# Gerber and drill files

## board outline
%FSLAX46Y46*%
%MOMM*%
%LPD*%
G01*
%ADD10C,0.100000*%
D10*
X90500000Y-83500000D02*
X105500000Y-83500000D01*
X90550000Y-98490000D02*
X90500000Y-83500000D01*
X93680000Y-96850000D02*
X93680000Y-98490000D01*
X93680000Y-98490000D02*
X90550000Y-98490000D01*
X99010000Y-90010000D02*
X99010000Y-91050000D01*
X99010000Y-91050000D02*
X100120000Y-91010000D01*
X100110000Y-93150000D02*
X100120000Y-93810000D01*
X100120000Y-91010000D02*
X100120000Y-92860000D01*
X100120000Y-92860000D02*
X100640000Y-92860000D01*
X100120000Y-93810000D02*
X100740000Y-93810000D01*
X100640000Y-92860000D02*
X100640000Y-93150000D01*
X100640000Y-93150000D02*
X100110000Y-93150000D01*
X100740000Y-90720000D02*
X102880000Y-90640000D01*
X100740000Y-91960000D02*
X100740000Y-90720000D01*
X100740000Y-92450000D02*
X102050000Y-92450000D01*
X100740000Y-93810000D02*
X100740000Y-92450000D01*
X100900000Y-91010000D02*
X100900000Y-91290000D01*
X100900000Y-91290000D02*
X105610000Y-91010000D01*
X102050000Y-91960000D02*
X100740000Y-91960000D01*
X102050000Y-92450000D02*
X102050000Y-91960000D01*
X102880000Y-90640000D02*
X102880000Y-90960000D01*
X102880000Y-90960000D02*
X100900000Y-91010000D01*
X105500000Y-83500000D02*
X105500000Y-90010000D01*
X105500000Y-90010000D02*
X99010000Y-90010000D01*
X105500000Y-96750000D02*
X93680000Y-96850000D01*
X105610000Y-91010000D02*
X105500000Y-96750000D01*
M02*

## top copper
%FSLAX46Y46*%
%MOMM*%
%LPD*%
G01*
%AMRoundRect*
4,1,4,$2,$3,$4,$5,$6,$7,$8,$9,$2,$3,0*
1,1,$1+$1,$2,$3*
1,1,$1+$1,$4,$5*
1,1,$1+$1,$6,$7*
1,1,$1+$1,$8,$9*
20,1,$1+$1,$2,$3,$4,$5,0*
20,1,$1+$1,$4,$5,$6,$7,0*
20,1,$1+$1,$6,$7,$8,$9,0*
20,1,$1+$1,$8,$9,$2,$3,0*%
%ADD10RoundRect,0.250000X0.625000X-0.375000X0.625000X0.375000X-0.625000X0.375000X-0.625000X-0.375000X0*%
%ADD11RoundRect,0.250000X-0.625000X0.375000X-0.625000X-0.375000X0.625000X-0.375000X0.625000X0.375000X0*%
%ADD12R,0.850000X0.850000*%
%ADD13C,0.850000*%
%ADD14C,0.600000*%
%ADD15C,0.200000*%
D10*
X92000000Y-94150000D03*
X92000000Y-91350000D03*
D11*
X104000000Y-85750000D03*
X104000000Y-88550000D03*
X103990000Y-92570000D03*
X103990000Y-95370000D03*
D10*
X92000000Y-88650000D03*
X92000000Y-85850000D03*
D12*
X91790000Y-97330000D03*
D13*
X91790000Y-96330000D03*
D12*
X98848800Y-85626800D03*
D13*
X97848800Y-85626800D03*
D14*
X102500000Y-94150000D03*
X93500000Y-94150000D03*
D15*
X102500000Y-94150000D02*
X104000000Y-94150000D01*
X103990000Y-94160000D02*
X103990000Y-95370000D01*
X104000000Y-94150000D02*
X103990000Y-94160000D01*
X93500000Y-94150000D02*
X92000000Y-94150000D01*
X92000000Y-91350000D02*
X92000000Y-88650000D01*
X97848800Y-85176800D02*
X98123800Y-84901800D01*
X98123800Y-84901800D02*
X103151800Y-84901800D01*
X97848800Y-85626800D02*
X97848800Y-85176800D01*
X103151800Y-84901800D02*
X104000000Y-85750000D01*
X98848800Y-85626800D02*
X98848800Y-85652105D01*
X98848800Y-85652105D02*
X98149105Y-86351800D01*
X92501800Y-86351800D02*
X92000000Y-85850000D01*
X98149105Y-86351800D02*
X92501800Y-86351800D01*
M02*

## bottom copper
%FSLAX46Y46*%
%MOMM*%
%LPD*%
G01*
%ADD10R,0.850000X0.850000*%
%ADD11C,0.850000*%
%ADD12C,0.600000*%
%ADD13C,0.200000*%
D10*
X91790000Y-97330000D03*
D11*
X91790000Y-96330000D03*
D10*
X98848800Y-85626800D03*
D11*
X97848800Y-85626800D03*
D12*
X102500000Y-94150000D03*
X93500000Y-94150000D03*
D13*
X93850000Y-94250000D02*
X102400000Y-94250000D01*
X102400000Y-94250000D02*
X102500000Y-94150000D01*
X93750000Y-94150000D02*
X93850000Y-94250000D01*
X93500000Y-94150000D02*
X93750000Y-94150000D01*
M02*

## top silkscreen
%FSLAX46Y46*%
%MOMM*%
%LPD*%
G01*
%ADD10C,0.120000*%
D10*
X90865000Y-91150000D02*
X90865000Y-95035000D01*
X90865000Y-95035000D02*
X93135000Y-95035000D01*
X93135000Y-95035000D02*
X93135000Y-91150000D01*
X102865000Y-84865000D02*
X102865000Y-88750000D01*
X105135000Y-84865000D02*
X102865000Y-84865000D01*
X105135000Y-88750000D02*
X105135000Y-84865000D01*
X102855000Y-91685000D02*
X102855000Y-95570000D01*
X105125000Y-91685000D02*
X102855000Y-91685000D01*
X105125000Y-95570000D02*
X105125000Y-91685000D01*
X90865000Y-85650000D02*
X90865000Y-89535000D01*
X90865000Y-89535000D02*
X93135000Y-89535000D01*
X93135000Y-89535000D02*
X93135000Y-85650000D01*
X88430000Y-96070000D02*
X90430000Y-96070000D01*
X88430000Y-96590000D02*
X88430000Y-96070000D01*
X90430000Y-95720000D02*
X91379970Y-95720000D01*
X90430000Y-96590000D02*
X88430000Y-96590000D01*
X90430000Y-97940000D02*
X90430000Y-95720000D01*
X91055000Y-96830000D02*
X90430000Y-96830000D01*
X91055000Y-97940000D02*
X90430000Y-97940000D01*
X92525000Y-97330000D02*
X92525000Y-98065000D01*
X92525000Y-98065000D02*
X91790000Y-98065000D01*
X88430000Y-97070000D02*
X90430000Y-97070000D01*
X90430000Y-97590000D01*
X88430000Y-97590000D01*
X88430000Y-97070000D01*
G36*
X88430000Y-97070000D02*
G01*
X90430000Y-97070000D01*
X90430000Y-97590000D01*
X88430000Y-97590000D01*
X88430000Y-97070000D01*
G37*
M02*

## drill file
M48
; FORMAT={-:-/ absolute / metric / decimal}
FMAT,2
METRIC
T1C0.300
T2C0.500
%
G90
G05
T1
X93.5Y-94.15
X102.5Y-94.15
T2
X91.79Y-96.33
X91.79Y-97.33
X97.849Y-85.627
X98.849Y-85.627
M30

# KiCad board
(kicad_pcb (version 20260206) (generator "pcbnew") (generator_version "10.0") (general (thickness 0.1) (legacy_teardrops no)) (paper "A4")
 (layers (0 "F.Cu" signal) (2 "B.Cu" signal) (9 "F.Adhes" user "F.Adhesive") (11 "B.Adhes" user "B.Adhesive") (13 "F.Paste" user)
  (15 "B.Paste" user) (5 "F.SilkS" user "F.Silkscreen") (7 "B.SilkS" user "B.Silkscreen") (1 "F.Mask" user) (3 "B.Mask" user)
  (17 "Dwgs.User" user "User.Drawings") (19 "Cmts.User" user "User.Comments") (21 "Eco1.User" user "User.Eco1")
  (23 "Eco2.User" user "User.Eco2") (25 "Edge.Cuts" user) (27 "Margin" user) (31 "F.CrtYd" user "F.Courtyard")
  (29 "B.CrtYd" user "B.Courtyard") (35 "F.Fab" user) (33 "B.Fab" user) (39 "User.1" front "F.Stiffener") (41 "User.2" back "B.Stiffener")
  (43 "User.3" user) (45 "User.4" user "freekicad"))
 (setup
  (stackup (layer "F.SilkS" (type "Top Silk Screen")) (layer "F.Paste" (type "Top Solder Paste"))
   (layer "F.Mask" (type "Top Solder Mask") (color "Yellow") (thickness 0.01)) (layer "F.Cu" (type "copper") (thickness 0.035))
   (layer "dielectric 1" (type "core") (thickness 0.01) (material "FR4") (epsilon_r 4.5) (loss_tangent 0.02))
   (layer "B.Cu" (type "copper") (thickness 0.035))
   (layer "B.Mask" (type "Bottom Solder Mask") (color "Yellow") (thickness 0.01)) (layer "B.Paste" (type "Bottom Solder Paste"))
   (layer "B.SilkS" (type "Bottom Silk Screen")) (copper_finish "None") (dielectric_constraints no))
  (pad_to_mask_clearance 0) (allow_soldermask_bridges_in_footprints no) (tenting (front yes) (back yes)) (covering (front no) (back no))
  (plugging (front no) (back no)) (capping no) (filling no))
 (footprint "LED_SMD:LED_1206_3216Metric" (layer "F.Cu") (at 92 92.75 90)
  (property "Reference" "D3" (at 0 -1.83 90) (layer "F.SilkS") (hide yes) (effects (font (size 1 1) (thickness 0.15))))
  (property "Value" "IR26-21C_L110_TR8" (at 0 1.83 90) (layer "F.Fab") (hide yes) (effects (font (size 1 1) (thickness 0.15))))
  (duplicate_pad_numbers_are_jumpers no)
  (fp_line (start 1.6 -1.135) (end -2.285 -1.135) (stroke (width 0.12) (type solid)) (layer "F.SilkS"))
  (fp_line (start -2.285 -1.135) (end -2.285 1.135) (stroke (width 0.12) (type solid)) (layer "F.SilkS"))
  (fp_line (start -2.285 1.135) (end 1.6 1.135) (stroke (width 0.12) (type solid)) (layer "F.SilkS"))
  (pad "1" smd roundrect (at -1.4 0 90) (size 1.25 1.75) (layers "F.Cu" "F.Mask" "F.Paste") (roundrect_rratio 0.2) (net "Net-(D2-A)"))
  (pad "2" smd roundrect (at 1.4 0 90) (size 1.25 1.75) (layers "F.Cu" "F.Mask" "F.Paste") (roundrect_rratio 0.2) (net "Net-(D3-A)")))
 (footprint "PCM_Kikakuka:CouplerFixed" (layer "F.Cu") (at 91.79 97.33 -90)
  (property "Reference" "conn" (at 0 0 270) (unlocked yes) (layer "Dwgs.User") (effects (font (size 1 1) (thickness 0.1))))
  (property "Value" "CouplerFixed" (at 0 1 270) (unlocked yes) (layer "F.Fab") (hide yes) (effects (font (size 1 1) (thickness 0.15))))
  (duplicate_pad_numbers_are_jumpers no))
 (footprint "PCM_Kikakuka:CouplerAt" (layer "F.Cu") (at 97.917 89.662)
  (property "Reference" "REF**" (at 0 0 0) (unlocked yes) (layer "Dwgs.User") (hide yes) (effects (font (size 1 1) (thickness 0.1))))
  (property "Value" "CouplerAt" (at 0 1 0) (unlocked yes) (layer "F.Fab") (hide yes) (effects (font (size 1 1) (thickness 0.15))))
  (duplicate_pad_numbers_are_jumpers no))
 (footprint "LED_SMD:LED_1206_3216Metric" (layer "F.Cu") (at 104 87.15 -90)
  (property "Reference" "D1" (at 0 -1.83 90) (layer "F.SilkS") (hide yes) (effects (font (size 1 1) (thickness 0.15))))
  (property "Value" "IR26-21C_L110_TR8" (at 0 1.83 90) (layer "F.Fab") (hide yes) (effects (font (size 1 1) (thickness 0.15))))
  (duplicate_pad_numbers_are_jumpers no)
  (fp_line (start -2.285 1.135) (end 1.6 1.135) (stroke (width 0.12) (type solid)) (layer "F.SilkS"))
  (fp_line (start -2.285 -1.135) (end -2.285 1.135) (stroke (width 0.12) (type solid)) (layer "F.SilkS"))
  (fp_line (start 1.6 -1.135) (end -2.285 -1.135) (stroke (width 0.12) (type solid)) (layer "F.SilkS"))
  (pad "1" smd roundrect (at -1.4 0 270) (size 1.25 1.75) (layers "F.Cu" "F.Mask" "F.Paste") (roundrect_rratio 0.2) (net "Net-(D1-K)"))
  (pad "2" smd roundrect (at 1.4 0 270) (size 1.25 1.75) (layers "F.Cu" "F.Mask" "F.Paste") (roundrect_rratio 0.2) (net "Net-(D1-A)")))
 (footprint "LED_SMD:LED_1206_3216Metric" (layer "F.Cu") (at 103.99 93.97 -90)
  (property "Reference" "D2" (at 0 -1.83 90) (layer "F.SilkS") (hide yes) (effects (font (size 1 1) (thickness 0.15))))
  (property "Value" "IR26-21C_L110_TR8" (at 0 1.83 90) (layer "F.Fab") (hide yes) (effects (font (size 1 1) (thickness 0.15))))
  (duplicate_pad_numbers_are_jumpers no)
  (fp_line (start -2.285 1.135) (end 1.6 1.135) (stroke (width 0.12) (type solid)) (layer "F.SilkS"))
  (fp_line (start -2.285 -1.135) (end -2.285 1.135) (stroke (width 0.12) (type solid)) (layer "F.SilkS"))
  (fp_line (start 1.6 -1.135) (end -2.285 -1.135) (stroke (width 0.12) (type solid)) (layer "F.SilkS"))
  (pad "1" smd roundrect (at -1.4 0 270) (size 1.25 1.75) (layers "F.Cu" "F.Mask" "F.Paste") (roundrect_rratio 0.2) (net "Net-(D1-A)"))
  (pad "2" smd roundrect (at 1.4 0 270) (size 1.25 1.75) (layers "F.Cu" "F.Mask" "F.Paste") (roundrect_rratio 0.2) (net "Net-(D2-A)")))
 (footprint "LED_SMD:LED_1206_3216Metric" (layer "F.Cu") (at 92 87.25 90)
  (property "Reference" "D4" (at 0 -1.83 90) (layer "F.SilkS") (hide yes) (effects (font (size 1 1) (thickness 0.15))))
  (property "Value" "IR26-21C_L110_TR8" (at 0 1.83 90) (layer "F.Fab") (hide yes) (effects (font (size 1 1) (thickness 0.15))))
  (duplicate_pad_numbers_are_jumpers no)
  (fp_line (start 1.6 -1.135) (end -2.285 -1.135) (stroke (width 0.12) (type solid)) (layer "F.SilkS"))
  (fp_line (start -2.285 -1.135) (end -2.285 1.135) (stroke (width 0.12) (type solid)) (layer "F.SilkS"))
  (fp_line (start -2.285 1.135) (end 1.6 1.135) (stroke (width 0.12) (type solid)) (layer "F.SilkS"))
  (pad "1" smd roundrect (at -1.4 0 90) (size 1.25 1.75) (layers "F.Cu" "F.Mask" "F.Paste") (roundrect_rratio 0.2) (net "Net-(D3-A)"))
  (pad "2" smd roundrect (at 1.4 0 90) (size 1.25 1.75) (layers "F.Cu" "F.Mask" "F.Paste") (roundrect_rratio 0.2) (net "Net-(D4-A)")))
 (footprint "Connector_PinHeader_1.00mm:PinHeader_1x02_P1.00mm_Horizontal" (layer "F.Cu") (at 91.79 97.33 180)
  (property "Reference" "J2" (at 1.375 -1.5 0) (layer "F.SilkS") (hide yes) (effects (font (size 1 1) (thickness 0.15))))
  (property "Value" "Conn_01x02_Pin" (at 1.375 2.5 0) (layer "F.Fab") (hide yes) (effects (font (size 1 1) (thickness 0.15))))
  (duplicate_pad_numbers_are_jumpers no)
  (fp_line (start 3.36 1.26) (end 1.36 1.26) (stroke (width 0.12) (type solid)) (layer "F.SilkS"))
  (fp_line (start 3.36 0.74) (end 3.36 1.26) (stroke (width 0.12) (type solid)) (layer "F.SilkS"))
  (fp_line (start 1.36 1.61) (end 0.41003 1.61) (stroke (width 0.12) (type solid)) (layer "F.SilkS"))
  (fp_line (start 1.36 0.74) (end 3.36 0.74) (stroke (width 0.12) (type solid)) (layer "F.SilkS"))
  (fp_line (start 1.36 -0.61) (end 1.36 1.61) (stroke (width 0.12) (type solid)) (layer "F.SilkS"))
  (fp_line (start 0.735 0.5) (end 1.36 0.5) (stroke (width 0.12) (type solid)) (layer "F.SilkS"))
  (fp_line (start 0.735 -0.61) (end 1.36 -0.61) (stroke (width 0.12) (type solid)) (layer "F.SilkS"))
  (fp_line (start -0.735 0) (end -0.735 -0.735) (stroke (width 0.12) (type solid)) (layer "F.SilkS"))
  (fp_line (start -0.735 -0.735) (end 0 -0.735) (stroke (width 0.12) (type solid)) (layer "F.SilkS"))
  (fp_rect (start 1.36 -0.26) (end 3.36 0.26) (stroke (width 0.12) (type solid)) (fill yes) (layer "F.SilkS"))
  (pad "1" thru_hole rect (at 0 0 180) (size 0.85 0.85) (drill 0.5) (layers "*.Cu" "*.Mask") (remove_unused_layers no))
  (pad "2" thru_hole circle (at 0 1 180) (size 0.85 0.85) (drill 0.5) (layers "*.Cu" "*.Mask") (remove_unused_layers no)))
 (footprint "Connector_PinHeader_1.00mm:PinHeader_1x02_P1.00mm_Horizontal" (layer "B.Cu") (at 98.8488 85.6268 90)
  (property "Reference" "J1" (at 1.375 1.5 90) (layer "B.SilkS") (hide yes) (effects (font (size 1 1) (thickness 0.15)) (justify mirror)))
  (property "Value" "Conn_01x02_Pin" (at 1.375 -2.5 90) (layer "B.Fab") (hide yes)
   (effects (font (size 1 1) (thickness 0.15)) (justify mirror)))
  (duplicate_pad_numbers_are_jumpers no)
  (pad "1" thru_hole rect (at 0 0 90) (size 0.85 0.85) (drill 0.5) (layers "*.Cu" "*.Mask") (remove_unused_layers no) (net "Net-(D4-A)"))
  (pad "2" thru_hole circle (at 0 -1 90) (size 0.85 0.85) (drill 0.5) (layers "*.Cu" "*.Mask") (remove_unused_layers no) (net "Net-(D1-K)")))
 (gr_line (start 90.5 83.5) (end 105.5 83.5) (stroke (width 0.1) (type default)) (layer "Edge.Cuts"))
 (gr_line (start 90.55 98.49) (end 90.5 83.5) (stroke (width 0.1) (type default)) (layer "Edge.Cuts"))
 (gr_line (start 93.68 96.85) (end 93.68 98.49) (stroke (width 0.1) (type default)) (layer "Edge.Cuts"))
 (gr_line (start 93.68 98.49) (end 90.55 98.49) (stroke (width 0.1) (type default)) (layer "Edge.Cuts"))
 (gr_line (start 99.01 90.01) (end 99.01 91.05) (stroke (width 0.1) (type default)) (layer "Edge.Cuts"))
 (gr_line (start 99.01 91.05) (end 100.12 91.01) (stroke (width 0.1) (type default)) (layer "Edge.Cuts"))
 (gr_line (start 100.11 93.15) (end 100.12 93.81) (stroke (width 0.1) (type default)) (layer "Edge.Cuts"))
 (gr_line (start 100.12 91.01) (end 100.12 92.86) (stroke (width 0.1) (type default)) (layer "Edge.Cuts"))
 (gr_line (start 100.12 92.86) (end 100.64 92.86) (stroke (width 0.1) (type default)) (layer "Edge.Cuts"))
 (gr_line (start 100.12 93.81) (end 100.74 93.81) (stroke (width 0.1) (type default)) (layer "Edge.Cuts"))
 (gr_line (start 100.64 92.86) (end 100.64 93.15) (stroke (width 0.1) (type default)) (layer "Edge.Cuts"))
 (gr_line (start 100.64 93.15) (end 100.11 93.15) (stroke (width 0.1) (type default)) (layer "Edge.Cuts"))
 (gr_line (start 100.74 90.72) (end 102.88 90.64) (stroke (width 0.1) (type default)) (layer "Edge.Cuts"))
 (gr_line (start 100.74 91.96) (end 100.74 90.72) (stroke (width 0.1) (type default)) (layer "Edge.Cuts"))
 (gr_line (start 100.74 92.45) (end 102.05 92.45) (stroke (width 0.1) (type default)) (layer "Edge.Cuts"))
 (gr_line (start 100.74 93.81) (end 100.74 92.45) (stroke (width 0.1) (type default)) (layer "Edge.Cuts"))
 (gr_line (start 100.9 91.01) (end 100.9 91.29) (stroke (width 0.1) (type default)) (layer "Edge.Cuts"))
 (gr_line (start 100.9 91.29) (end 105.61 91.01) (stroke (width 0.1) (type default)) (layer "Edge.Cuts"))
 (gr_line (start 102.05 91.96) (end 100.74 91.96) (stroke (width 0.1) (type default)) (layer "Edge.Cuts"))
 (gr_line (start 102.05 92.45) (end 102.05 91.96) (stroke (width 0.1) (type default)) (layer "Edge.Cuts"))
 (gr_line (start 102.88 90.64) (end 102.88 90.96) (stroke (width 0.1) (type default)) (layer "Edge.Cuts"))
 (gr_line (start 102.88 90.96) (end 100.9 91.01) (stroke (width 0.1) (type default)) (layer "Edge.Cuts"))
 (gr_line (start 105.5 83.5) (end 105.5 90.01) (stroke (width 0.1) (type default)) (layer "Edge.Cuts"))
 (gr_line (start 105.5 90.01) (end 99.01 90.01) (stroke (width 0.1) (type default)) (layer "Edge.Cuts"))
 (gr_line (start 105.5 96.75) (end 93.68 96.85) (stroke (width 0.1) (type default)) (layer "Edge.Cuts"))
 (gr_line (start 105.61 91.01) (end 105.5 96.75) (stroke (width 0.1) (type default)) (layer "Edge.Cuts"))
 (segment (start 102.5 94.15) (end 104 94.15) (width 0.2) (layer "F.Cu") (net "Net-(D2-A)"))
 (segment (start 103.99 94.16) (end 103.99 95.37) (width 0.2) (layer "F.Cu") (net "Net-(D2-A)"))
 (segment (start 104 94.15) (end 103.99 94.16) (width 0.2) (layer "F.Cu") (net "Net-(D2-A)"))
 (segment (start 93.5 94.15) (end 92 94.15) (width 0.2) (layer "F.Cu") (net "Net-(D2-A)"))
 (via (at 102.5 94.15) (size 0.6) (drill 0.3) (layers "F.Cu" "B.Cu") (capping no) (covering (front no) (back no))
  (plugging (front no) (back no)) (filling no) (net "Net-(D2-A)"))
 (via (at 93.5 94.15) (size 0.6) (drill 0.3) (layers "F.Cu" "B.Cu") (capping no) (covering (front no) (back no))
  (plugging (front no) (back no)) (filling no) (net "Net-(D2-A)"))
 (segment (start 93.85 94.25) (end 102.4 94.25) (width 0.2) (layer "B.Cu") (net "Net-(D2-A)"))
 (segment (start 102.4 94.25) (end 102.5 94.15) (width 0.2) (layer "B.Cu") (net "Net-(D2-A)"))
 (segment (start 93.75 94.15) (end 93.85 94.25) (width 0.2) (layer "B.Cu") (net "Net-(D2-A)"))
 (segment (start 93.5 94.15) (end 93.75 94.15) (width 0.2) (layer "B.Cu") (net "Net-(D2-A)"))
 (segment (start 92 91.35) (end 92 88.65) (width 0.2) (layer "F.Cu") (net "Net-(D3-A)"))
 (segment (start 97.8488 85.1768) (end 98.1238 84.9018) (width 0.2) (layer "F.Cu") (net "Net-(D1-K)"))
 (segment (start 98.1238 84.9018) (end 103.1518 84.9018) (width 0.2) (layer "F.Cu") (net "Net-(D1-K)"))
 (segment (start 97.8488 85.6268) (end 97.8488 85.1768) (width 0.2) (layer "F.Cu") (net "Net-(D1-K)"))
 (segment (start 103.1518 84.9018) (end 104 85.75) (width 0.2) (layer "F.Cu") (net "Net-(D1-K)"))
 (segment (start 98.8488 85.6268) (end 98.8488 85.652105) (width 0.2) (layer "F.Cu") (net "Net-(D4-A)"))
 (segment (start 98.8488 85.652105) (end 98.149105 86.3518) (width 0.2) (layer "F.Cu") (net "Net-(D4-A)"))
 (segment (start 92.5018 86.3518) (end 92 85.85) (width 0.2) (layer "F.Cu") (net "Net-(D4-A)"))
 (segment (start 98.149105 86.3518) (end 92.5018 86.3518) (width 0.2) (layer "F.Cu") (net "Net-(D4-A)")))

